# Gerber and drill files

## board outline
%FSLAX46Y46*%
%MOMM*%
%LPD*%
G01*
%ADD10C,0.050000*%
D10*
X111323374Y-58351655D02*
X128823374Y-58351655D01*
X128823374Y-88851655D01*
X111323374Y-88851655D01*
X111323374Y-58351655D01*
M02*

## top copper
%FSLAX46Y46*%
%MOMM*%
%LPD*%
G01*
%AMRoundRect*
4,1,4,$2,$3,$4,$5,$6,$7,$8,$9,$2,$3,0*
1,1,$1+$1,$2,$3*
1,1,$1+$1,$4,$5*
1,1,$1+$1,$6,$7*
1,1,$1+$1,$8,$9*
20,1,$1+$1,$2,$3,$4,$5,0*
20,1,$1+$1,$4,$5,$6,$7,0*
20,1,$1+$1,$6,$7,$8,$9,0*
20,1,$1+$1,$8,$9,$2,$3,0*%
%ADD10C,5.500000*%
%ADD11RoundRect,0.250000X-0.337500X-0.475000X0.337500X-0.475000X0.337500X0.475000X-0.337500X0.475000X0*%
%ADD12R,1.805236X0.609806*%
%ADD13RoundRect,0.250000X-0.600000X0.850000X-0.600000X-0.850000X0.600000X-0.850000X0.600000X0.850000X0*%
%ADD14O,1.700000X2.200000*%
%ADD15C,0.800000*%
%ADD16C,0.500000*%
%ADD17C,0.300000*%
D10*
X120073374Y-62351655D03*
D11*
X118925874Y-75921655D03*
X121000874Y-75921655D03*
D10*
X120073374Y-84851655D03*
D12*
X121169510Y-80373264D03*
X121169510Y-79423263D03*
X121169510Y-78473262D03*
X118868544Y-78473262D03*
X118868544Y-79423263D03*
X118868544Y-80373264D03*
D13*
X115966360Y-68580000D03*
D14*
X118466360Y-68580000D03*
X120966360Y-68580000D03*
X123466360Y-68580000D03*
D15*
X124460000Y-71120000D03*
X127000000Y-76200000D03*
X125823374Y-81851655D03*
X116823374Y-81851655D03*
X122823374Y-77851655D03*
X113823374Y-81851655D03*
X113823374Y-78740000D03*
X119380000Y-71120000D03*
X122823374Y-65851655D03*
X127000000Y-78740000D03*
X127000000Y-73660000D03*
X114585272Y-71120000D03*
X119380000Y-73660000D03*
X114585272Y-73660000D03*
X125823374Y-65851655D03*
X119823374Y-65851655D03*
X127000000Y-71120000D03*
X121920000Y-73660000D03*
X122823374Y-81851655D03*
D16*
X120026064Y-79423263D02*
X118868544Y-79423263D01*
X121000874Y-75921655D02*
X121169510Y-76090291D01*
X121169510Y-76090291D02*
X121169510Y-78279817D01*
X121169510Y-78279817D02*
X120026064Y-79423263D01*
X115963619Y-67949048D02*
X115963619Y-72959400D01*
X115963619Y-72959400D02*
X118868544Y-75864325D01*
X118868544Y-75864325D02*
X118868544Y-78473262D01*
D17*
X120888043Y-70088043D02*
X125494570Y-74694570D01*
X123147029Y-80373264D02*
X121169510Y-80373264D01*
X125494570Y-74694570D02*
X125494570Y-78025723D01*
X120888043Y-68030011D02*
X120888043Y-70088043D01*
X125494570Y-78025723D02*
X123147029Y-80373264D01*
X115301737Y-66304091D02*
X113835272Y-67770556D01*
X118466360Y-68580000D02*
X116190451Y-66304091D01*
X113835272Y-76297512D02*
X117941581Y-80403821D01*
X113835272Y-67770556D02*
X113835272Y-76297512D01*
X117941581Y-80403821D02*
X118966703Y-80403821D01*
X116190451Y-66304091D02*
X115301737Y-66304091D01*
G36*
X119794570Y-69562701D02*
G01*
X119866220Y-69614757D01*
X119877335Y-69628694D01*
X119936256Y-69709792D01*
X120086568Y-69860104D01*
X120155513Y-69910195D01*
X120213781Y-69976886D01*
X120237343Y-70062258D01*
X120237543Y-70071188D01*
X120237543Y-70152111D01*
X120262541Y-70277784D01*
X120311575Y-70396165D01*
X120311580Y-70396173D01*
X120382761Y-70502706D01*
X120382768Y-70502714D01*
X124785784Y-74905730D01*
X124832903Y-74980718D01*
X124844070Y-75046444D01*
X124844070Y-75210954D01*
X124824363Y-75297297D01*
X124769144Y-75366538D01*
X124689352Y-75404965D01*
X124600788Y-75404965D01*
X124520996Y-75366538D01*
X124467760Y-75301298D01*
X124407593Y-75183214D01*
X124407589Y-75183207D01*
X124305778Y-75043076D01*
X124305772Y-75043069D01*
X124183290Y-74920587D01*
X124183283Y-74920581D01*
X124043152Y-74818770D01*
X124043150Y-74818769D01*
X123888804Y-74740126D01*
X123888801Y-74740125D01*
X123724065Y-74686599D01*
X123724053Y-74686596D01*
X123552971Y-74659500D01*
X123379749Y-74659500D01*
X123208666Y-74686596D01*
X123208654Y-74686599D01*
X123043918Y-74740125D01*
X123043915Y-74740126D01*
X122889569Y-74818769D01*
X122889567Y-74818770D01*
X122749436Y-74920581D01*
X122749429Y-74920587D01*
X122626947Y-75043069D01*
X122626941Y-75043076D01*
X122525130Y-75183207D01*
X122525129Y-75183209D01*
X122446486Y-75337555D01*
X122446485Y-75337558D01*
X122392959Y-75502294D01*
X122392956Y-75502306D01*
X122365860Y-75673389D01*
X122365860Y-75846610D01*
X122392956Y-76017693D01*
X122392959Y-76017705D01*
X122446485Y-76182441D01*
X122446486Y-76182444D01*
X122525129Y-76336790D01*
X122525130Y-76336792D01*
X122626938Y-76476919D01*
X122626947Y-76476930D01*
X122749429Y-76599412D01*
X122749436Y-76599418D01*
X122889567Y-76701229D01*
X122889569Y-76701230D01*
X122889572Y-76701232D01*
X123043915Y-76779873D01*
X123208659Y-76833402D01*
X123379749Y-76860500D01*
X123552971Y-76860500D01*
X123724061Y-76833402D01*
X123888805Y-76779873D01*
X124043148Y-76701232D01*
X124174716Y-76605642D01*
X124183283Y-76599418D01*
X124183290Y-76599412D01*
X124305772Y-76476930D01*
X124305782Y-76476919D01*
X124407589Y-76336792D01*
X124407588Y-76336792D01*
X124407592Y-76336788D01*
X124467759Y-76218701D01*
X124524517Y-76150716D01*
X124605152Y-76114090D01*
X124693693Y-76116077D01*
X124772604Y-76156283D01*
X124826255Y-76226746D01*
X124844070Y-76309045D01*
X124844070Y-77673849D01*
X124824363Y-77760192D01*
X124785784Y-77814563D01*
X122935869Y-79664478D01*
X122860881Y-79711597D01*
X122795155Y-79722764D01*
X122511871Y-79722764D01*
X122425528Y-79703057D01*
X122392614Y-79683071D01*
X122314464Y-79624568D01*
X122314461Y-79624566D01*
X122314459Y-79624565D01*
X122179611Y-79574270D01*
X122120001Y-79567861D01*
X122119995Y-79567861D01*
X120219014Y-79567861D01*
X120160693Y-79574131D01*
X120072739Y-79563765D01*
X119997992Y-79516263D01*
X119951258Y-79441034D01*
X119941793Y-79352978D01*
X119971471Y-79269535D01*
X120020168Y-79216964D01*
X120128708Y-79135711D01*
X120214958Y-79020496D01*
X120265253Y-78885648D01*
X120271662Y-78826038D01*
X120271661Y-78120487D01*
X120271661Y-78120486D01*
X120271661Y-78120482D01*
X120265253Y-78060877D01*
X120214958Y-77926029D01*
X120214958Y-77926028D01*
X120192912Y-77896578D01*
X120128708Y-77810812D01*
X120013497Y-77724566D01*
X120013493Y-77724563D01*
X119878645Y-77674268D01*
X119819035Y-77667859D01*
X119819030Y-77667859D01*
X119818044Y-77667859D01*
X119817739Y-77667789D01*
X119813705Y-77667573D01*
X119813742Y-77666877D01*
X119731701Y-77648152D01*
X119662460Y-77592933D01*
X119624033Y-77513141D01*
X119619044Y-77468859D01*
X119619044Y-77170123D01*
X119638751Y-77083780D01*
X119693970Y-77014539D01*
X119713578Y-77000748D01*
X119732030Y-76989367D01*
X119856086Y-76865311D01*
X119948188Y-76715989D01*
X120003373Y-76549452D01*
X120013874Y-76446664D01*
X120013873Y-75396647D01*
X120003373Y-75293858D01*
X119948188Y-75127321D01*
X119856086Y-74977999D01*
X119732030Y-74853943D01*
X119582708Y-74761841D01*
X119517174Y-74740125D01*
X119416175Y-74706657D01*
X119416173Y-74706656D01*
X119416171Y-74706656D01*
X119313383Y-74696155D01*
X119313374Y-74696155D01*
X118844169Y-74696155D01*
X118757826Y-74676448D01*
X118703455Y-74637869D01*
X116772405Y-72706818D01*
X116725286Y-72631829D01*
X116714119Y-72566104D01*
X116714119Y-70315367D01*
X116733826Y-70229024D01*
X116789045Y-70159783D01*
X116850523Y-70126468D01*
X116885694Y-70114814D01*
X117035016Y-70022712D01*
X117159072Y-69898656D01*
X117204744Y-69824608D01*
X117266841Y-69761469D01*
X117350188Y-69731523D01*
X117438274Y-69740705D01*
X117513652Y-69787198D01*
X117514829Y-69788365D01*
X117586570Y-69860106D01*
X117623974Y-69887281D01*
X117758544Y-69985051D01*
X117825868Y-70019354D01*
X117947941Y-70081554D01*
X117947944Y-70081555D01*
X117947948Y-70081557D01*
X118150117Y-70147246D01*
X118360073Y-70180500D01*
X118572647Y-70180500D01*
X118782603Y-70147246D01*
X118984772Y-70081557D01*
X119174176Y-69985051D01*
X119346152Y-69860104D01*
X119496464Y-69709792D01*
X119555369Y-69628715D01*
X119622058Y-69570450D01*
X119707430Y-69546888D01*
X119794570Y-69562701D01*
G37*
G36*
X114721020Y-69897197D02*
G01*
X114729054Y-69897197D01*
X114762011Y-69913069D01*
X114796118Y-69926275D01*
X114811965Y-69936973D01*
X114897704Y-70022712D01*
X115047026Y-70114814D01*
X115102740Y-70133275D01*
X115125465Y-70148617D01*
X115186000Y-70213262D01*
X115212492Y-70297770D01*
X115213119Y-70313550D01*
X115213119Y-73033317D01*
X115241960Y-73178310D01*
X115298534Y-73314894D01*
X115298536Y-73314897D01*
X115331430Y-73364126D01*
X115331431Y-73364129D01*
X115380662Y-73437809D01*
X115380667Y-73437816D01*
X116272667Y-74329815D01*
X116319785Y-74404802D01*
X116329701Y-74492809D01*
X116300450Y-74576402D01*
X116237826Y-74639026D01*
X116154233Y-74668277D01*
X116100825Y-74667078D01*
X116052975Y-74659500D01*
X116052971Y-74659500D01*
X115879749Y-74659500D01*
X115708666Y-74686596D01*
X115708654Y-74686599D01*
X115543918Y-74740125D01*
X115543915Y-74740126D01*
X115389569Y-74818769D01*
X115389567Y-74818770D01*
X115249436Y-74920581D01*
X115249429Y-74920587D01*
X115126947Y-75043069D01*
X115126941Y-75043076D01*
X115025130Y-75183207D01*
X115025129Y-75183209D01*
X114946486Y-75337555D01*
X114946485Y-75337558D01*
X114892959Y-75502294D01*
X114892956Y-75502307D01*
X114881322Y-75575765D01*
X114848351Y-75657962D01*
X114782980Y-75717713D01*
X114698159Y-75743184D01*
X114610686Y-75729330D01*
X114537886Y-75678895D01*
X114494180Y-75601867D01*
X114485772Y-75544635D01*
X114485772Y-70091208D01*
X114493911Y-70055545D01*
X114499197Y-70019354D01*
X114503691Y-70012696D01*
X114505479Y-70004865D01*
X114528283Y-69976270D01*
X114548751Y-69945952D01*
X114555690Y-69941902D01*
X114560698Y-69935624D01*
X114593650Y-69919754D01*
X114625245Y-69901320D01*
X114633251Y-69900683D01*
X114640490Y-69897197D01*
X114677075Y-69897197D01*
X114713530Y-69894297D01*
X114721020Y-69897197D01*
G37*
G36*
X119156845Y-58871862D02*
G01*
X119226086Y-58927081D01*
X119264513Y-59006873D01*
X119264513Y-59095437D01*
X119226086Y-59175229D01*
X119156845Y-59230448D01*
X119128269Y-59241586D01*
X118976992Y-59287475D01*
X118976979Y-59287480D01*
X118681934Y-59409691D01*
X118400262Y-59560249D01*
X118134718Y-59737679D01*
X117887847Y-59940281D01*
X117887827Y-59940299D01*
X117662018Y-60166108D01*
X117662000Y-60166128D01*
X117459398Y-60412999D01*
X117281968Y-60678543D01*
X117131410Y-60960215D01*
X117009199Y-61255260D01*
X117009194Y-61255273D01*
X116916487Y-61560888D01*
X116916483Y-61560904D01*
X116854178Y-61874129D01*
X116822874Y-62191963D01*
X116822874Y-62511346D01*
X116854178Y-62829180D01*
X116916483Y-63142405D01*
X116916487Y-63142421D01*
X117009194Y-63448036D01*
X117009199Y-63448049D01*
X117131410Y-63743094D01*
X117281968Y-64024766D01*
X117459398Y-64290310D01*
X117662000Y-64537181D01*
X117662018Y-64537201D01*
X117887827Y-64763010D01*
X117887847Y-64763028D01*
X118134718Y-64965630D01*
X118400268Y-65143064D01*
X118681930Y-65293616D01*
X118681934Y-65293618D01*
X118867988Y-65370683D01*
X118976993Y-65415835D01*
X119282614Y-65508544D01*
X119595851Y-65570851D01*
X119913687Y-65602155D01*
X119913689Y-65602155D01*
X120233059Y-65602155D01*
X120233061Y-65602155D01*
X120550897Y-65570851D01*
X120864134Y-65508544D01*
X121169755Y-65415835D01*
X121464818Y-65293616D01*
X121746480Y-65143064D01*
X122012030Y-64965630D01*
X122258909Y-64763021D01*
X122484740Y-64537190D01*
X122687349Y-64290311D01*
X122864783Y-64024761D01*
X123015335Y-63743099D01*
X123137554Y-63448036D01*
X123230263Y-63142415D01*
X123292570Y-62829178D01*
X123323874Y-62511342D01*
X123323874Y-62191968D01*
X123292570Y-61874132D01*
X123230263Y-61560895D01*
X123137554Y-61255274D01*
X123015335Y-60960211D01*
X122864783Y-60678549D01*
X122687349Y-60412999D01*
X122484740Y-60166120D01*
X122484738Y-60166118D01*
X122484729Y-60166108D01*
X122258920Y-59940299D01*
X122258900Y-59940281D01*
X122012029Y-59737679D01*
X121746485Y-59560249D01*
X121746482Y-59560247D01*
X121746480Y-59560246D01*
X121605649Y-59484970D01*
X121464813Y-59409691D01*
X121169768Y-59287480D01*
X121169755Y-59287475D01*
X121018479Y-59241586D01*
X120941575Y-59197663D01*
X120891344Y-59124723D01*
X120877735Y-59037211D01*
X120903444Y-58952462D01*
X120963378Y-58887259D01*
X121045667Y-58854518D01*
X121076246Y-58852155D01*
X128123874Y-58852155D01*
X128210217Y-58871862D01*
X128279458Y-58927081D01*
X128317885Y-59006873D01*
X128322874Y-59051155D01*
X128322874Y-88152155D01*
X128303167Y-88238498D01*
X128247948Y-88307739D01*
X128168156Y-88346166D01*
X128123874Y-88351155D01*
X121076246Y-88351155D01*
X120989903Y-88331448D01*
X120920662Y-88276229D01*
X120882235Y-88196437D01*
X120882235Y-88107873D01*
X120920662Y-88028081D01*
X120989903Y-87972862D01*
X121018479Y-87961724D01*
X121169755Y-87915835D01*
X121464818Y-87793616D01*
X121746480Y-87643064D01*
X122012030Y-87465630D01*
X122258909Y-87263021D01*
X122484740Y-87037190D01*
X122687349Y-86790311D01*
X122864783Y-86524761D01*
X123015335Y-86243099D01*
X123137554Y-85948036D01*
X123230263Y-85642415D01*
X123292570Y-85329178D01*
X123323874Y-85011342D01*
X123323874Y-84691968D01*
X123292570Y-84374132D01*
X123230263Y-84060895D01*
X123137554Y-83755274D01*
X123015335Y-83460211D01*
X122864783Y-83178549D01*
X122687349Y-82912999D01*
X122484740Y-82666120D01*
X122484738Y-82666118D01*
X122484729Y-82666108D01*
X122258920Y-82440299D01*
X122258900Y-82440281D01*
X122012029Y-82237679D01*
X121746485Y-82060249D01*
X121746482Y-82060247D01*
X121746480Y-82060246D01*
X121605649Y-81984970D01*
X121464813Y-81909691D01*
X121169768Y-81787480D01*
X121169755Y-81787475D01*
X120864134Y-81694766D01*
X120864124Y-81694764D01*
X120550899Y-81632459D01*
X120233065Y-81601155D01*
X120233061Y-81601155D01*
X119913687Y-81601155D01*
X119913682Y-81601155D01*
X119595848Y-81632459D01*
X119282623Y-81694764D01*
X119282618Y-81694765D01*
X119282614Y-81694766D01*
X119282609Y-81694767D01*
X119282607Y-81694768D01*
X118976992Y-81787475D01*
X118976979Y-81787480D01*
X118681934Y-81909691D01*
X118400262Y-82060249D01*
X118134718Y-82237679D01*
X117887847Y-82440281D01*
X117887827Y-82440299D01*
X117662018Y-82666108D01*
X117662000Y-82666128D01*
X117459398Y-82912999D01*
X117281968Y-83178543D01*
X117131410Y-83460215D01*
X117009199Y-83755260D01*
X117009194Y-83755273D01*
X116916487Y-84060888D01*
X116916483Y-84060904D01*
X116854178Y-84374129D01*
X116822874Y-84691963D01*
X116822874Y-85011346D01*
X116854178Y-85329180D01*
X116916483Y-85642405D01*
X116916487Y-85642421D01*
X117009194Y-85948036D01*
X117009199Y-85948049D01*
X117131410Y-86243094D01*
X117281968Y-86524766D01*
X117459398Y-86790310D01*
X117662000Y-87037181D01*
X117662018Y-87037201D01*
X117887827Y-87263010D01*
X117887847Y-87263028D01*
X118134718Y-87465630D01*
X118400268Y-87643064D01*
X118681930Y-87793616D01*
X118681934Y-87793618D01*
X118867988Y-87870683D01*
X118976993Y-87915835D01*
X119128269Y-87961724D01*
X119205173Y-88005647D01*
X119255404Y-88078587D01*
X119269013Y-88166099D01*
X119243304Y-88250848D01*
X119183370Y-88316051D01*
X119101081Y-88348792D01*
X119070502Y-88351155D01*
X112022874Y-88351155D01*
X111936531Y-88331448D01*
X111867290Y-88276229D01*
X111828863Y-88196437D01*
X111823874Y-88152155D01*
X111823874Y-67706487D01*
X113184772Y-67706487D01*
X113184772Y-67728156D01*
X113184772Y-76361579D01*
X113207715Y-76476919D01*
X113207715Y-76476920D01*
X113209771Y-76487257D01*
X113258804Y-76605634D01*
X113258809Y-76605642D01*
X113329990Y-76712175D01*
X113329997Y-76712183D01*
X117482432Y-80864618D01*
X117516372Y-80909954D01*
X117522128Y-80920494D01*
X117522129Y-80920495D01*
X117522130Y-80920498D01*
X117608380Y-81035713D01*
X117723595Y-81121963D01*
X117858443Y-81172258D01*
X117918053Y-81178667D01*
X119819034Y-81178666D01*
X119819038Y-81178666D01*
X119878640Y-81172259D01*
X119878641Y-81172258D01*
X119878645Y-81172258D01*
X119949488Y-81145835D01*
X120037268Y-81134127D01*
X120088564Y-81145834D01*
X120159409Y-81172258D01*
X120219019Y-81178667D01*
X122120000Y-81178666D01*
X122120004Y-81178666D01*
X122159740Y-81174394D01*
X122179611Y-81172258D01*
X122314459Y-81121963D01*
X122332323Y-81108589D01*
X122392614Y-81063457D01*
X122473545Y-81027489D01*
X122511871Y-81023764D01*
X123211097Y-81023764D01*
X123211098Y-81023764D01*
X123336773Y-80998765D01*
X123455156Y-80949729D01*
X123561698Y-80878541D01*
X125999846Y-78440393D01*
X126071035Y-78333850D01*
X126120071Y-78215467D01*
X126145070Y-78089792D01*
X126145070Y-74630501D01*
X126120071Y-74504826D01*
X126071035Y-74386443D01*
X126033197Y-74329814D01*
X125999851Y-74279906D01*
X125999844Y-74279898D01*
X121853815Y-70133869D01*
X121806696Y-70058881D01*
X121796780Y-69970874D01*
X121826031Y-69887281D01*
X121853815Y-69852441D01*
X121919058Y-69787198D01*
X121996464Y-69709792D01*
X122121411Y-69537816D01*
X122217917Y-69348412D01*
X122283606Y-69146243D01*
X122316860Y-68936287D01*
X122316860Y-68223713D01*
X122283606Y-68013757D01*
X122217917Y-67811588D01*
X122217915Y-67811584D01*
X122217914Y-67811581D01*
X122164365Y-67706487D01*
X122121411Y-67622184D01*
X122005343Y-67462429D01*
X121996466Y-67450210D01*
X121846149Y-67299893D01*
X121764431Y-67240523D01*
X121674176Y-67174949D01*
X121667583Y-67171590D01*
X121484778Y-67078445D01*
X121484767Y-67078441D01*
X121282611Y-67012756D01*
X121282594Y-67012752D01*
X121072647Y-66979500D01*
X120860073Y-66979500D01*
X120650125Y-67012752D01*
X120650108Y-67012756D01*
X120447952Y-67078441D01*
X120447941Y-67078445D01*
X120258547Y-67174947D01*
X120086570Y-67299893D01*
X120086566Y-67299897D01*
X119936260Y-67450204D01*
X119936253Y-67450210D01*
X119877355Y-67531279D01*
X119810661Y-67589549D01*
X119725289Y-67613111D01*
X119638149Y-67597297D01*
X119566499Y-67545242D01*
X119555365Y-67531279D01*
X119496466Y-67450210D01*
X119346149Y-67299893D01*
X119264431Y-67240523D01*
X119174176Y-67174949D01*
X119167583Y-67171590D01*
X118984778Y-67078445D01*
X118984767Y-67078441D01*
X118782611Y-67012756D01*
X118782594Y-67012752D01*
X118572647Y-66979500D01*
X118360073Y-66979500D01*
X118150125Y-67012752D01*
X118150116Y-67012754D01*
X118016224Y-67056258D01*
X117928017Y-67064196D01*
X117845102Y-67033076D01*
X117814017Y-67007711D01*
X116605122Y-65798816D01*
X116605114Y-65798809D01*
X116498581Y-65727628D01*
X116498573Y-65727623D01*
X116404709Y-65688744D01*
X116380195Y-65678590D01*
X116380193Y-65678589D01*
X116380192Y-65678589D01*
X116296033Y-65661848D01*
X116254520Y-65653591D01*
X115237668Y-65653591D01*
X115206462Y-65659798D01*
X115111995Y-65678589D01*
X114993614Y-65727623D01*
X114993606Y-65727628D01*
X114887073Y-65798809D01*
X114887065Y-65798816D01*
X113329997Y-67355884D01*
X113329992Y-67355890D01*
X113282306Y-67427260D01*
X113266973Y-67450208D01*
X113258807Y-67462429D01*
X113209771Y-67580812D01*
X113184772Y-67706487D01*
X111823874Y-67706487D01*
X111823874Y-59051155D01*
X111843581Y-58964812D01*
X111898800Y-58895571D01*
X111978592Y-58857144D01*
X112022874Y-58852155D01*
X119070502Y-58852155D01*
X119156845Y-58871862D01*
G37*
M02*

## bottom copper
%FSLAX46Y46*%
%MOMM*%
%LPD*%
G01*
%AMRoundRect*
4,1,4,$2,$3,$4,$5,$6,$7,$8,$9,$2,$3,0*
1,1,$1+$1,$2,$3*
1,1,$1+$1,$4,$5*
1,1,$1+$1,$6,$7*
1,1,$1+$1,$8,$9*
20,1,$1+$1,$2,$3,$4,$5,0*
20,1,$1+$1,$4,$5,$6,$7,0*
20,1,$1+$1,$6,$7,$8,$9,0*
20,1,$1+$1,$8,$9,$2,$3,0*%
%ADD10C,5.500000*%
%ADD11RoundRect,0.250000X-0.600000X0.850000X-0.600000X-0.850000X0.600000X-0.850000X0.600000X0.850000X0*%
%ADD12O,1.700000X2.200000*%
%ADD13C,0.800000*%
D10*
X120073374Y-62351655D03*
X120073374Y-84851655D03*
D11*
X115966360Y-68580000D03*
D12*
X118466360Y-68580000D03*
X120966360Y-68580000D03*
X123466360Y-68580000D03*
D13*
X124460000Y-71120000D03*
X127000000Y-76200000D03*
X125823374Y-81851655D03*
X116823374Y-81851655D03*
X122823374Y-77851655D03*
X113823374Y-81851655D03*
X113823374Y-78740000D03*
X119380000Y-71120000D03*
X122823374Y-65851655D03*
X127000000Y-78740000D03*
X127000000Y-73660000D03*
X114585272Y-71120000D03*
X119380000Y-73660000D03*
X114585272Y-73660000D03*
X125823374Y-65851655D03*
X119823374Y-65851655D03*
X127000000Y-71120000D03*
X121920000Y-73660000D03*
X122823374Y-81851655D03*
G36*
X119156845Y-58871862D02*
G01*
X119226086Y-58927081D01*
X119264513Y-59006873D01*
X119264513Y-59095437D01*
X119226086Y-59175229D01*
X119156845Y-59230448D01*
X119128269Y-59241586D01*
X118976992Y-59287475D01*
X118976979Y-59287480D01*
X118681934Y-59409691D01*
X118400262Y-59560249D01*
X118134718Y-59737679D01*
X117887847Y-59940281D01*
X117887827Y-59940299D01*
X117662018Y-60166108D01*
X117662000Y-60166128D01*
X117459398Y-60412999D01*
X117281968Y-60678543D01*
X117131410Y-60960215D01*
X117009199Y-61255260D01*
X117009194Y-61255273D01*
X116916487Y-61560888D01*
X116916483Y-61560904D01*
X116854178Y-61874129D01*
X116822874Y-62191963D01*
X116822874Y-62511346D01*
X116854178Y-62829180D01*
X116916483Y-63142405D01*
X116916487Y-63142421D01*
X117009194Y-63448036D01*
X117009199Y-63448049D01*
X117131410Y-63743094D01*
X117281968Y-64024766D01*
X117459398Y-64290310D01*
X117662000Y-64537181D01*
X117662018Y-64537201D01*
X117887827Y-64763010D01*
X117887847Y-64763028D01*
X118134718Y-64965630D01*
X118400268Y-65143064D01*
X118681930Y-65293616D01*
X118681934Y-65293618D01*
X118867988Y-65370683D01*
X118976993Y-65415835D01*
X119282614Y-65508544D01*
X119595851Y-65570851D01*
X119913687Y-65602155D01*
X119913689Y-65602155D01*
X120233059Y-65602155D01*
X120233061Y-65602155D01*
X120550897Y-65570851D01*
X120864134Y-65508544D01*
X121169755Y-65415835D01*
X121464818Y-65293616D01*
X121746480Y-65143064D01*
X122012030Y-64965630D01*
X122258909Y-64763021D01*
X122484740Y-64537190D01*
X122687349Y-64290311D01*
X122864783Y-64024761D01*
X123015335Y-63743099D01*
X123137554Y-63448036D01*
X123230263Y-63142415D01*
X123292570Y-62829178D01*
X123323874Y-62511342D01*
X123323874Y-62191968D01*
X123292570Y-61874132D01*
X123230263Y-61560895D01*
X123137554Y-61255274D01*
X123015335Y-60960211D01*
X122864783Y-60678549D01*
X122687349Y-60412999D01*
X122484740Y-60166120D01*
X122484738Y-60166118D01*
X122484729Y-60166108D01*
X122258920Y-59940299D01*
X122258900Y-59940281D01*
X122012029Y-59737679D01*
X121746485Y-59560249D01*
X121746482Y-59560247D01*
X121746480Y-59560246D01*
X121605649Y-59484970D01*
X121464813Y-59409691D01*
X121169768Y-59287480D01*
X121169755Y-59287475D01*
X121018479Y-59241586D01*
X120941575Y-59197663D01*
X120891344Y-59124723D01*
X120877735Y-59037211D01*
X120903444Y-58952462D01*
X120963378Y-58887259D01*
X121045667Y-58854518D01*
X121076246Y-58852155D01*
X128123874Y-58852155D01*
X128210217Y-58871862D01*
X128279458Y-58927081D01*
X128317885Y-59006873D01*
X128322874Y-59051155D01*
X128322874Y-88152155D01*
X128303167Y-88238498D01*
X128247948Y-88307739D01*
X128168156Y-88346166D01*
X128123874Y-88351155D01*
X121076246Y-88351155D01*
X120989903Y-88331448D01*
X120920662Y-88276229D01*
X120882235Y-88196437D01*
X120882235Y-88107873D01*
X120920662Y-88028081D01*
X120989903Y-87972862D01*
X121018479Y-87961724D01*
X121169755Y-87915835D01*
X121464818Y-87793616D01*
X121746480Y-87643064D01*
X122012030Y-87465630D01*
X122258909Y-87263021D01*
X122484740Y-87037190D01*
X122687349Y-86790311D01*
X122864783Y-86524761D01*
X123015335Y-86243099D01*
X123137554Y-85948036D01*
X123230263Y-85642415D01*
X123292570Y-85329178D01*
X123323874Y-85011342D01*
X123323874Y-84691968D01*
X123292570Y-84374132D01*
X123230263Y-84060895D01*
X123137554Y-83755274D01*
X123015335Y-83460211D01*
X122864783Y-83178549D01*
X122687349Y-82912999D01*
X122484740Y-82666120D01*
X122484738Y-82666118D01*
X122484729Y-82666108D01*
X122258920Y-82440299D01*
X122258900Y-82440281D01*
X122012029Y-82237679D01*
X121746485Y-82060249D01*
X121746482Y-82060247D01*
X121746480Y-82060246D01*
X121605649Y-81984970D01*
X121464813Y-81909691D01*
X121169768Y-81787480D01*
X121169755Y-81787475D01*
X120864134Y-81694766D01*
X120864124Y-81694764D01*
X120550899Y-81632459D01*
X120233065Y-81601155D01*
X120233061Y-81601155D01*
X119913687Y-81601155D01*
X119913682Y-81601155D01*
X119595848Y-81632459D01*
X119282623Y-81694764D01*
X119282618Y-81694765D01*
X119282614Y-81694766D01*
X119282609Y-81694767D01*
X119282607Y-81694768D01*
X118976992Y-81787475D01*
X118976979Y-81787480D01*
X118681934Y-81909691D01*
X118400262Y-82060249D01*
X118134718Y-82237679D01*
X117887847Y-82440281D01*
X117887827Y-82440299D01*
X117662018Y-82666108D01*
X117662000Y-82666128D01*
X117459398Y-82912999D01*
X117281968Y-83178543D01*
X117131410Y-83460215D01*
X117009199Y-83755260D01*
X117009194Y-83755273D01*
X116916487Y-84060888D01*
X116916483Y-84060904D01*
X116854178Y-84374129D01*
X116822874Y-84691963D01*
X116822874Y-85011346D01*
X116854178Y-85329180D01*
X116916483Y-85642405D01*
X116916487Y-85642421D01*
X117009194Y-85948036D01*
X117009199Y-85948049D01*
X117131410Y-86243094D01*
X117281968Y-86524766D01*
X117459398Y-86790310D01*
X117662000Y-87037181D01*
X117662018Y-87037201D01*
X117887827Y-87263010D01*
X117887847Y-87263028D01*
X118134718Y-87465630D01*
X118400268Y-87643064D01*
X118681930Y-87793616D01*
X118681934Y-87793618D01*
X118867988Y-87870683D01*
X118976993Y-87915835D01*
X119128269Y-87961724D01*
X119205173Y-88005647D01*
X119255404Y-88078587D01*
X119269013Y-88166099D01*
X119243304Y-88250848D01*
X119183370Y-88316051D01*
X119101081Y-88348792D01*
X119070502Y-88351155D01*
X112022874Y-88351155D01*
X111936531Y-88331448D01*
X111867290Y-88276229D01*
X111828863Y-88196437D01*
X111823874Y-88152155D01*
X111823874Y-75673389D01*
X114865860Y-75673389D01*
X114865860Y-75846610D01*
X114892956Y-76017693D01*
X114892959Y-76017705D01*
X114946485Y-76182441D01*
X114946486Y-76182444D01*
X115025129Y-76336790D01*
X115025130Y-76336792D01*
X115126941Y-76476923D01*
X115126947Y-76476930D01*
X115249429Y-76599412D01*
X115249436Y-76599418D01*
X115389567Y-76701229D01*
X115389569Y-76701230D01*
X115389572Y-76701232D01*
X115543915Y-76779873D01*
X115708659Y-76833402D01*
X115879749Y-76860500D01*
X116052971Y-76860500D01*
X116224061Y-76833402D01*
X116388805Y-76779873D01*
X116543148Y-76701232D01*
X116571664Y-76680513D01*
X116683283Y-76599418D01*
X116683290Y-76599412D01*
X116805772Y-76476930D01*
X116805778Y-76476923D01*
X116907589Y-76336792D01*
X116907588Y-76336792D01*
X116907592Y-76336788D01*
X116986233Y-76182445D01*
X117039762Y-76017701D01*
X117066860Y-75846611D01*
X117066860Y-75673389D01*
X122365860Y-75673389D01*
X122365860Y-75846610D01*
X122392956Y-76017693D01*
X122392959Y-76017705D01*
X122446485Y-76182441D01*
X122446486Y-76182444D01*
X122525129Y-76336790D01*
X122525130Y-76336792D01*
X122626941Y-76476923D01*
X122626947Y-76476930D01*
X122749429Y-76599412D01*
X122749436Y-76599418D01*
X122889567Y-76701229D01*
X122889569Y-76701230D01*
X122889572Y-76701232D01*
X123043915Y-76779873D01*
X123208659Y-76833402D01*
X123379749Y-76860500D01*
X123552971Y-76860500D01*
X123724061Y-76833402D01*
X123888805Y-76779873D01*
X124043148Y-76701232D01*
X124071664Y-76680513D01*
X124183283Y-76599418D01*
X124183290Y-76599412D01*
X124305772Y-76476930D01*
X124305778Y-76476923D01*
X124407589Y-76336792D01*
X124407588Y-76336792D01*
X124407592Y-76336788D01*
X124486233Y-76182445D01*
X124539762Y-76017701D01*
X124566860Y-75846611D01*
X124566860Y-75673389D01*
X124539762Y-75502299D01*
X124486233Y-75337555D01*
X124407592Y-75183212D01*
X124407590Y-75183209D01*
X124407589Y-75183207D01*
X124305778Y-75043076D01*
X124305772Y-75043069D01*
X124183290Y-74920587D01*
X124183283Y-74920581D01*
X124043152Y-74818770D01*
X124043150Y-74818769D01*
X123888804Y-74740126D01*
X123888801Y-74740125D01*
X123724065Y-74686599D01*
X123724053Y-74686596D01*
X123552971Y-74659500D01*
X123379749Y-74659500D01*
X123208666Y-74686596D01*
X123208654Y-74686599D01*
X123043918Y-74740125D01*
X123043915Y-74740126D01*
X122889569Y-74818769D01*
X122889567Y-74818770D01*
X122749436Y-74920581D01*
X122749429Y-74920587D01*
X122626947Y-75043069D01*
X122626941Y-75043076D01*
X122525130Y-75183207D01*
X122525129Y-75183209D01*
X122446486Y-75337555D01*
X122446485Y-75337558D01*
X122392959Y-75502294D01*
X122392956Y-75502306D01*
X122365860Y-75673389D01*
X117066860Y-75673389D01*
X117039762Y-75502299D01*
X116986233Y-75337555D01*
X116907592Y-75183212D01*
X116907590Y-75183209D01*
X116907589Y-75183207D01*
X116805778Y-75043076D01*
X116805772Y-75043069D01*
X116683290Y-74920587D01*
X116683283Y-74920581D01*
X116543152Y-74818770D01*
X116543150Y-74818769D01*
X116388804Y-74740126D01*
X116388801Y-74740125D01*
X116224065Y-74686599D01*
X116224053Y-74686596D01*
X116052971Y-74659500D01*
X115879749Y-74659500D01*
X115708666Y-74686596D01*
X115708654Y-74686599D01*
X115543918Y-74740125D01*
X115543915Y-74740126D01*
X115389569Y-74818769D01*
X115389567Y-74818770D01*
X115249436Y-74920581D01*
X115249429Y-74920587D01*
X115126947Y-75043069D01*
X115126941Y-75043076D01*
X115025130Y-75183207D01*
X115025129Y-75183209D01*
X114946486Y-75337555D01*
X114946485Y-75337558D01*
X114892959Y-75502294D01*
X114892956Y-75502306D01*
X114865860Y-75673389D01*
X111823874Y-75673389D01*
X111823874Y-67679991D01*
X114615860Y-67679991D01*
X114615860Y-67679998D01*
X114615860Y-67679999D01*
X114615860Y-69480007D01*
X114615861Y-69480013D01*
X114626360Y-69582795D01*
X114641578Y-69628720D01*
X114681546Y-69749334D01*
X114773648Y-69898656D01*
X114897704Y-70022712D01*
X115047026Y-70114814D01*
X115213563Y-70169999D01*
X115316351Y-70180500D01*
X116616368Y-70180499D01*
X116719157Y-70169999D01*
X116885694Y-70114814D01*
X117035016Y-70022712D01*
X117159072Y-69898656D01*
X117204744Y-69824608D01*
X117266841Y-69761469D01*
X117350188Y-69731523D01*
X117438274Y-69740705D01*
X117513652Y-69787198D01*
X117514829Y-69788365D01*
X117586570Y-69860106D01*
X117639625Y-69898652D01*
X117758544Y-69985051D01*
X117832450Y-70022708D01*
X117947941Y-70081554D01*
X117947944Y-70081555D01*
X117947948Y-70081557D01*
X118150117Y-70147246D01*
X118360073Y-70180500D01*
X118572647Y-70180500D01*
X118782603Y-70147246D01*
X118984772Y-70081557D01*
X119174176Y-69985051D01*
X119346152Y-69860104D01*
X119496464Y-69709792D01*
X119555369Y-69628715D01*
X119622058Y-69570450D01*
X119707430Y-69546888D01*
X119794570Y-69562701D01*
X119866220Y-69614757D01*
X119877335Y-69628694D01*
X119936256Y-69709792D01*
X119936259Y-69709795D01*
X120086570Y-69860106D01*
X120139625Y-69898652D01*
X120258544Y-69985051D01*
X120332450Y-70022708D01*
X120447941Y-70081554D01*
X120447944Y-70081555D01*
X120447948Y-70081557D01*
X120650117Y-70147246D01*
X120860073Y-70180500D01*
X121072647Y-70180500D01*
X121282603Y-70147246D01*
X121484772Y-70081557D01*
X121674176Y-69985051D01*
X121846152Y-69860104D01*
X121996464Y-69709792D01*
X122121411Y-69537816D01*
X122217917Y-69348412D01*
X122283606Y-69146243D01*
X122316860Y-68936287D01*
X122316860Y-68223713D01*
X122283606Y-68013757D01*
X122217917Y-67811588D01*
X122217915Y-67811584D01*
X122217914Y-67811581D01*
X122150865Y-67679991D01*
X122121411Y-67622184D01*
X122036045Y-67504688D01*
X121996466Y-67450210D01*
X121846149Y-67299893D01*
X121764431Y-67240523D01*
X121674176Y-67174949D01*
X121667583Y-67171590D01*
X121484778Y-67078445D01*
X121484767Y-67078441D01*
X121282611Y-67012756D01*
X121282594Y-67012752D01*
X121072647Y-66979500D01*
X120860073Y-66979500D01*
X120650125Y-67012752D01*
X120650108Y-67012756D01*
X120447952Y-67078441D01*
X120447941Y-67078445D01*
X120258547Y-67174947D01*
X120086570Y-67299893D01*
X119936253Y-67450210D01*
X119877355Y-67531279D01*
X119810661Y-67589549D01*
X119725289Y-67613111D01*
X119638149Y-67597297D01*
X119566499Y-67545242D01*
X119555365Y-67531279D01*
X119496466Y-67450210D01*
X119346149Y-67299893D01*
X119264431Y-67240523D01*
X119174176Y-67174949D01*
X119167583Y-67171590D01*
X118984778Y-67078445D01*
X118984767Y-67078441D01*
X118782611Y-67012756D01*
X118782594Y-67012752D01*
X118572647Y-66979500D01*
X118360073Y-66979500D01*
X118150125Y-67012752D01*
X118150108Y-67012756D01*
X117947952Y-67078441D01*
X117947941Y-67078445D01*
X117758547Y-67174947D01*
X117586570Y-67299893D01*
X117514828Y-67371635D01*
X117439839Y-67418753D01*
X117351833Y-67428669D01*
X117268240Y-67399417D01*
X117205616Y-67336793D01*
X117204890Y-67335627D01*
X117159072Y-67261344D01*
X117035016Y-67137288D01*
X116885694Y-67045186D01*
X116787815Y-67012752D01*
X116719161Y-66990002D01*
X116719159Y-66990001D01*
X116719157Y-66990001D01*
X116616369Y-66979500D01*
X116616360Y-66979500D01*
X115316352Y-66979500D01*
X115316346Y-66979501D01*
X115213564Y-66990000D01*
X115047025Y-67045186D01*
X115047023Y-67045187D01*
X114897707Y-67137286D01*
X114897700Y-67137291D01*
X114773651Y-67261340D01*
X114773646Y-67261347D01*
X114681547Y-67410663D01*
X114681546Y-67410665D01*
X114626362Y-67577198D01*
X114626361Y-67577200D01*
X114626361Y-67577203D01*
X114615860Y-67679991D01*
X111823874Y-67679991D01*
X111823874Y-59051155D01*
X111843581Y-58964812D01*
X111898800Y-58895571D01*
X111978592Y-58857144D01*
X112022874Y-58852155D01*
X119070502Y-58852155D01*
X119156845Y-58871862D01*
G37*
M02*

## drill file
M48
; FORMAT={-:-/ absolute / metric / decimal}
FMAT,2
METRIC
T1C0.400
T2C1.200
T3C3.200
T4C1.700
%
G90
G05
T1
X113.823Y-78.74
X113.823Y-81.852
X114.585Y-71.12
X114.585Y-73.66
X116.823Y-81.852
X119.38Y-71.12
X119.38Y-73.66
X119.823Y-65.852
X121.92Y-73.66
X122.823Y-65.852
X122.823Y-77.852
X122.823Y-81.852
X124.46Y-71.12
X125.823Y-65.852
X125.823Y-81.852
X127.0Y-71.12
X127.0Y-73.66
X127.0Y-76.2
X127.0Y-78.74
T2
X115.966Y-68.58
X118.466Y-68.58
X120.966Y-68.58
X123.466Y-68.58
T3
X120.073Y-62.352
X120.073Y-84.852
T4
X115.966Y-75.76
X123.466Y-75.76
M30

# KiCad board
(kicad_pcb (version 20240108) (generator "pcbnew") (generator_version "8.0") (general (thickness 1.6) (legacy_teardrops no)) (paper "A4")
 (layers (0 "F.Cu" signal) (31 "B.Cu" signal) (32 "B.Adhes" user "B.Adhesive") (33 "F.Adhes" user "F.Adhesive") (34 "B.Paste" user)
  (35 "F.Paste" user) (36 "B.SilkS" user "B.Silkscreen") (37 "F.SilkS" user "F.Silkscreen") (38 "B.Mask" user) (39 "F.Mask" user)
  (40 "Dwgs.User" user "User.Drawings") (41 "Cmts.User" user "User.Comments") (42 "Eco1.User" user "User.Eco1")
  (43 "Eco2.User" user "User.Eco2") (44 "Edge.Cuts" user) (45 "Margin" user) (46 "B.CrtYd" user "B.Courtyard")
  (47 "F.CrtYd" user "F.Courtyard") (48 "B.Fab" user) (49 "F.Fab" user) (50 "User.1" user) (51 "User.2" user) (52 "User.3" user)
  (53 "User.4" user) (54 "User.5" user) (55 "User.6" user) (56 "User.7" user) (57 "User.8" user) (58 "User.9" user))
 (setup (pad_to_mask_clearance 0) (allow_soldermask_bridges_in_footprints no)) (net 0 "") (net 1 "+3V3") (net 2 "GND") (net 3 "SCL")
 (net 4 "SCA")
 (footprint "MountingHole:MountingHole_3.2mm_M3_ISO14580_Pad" (layer "F.Cu") (at 120.073374 62.351655)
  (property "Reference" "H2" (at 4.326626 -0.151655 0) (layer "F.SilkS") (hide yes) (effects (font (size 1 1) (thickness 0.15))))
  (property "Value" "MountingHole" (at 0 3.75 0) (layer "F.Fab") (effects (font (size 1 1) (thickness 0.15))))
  (pad "1" thru_hole circle (at 0 0) (size 5.5 5.5) (drill 3.2) (layers "*.Cu" "*.Mask") (remove_unused_layers no)))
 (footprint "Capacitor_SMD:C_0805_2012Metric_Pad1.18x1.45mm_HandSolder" (layer "F.Cu") (at 119.963374 75.921655)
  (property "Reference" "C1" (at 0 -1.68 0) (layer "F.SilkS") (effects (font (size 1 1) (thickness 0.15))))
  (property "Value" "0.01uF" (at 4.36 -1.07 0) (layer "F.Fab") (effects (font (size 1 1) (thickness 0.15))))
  (pad "1" smd roundrect (at -1.0375 0) (size 1.175 1.45) (layers "F.Cu" "F.Paste" "F.Mask") (roundrect_rratio 0.212766) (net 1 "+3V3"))
  (pad "2" smd roundrect (at 1.0375 0) (size 1.175 1.45) (layers "F.Cu" "F.Paste" "F.Mask") (roundrect_rratio 0.212766) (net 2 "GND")))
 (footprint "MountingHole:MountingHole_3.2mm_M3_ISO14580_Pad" (layer "F.Cu") (at 120.073374 84.851655)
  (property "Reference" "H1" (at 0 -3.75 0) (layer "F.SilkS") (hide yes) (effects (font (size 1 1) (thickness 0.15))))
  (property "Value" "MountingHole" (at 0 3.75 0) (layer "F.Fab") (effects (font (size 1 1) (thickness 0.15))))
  (pad "1" thru_hole circle (at 0 0) (size 5.5 5.5) (drill 3.2) (layers "*.Cu" "*.Mask") (remove_unused_layers no)))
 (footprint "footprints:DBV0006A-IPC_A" (layer "F.Cu") (at 120.019027 79.423263 180)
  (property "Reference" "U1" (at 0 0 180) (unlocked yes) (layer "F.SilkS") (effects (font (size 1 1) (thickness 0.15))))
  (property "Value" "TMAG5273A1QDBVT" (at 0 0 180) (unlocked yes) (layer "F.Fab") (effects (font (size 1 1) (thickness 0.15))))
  (pad "1" smd rect (at -1.150483 -0.950001 180) (size 1.805236 0.609806) (layers "F.Cu" "F.Paste" "F.Mask") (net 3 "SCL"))
  (pad "2" smd rect (at -1.150483 0 180) (size 1.805236 0.609806) (layers "F.Cu" "F.Paste" "F.Mask") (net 2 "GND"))
  (pad "3" smd rect (at -1.150483 0.950001 180) (size 1.805236 0.609806) (layers "F.Cu" "F.Paste" "F.Mask") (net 2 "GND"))
  (pad "4" smd rect (at 1.150483 0.950001 180) (size 1.805236 0.609806) (layers "F.Cu" "F.Paste" "F.Mask") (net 1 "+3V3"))
  (pad "5" smd rect (at 1.150483 0 180) (size 1.805236 0.609806) (layers "F.Cu" "F.Paste" "F.Mask") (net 2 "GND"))
  (pad "6" smd rect (at 1.150483 -0.950001 180) (size 1.805236 0.609806) (layers "F.Cu" "F.Paste" "F.Mask") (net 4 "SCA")))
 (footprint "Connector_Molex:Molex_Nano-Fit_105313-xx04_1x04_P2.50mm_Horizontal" (layer "B.Cu") (at 115.96636 68.58 -90)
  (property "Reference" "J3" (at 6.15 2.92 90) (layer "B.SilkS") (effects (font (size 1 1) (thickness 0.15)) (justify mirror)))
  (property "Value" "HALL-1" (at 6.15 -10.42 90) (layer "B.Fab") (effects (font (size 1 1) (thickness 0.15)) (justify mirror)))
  (pad "" np_thru_hole circle (at 7.18 -7.5 270) (size 1.7 1.7) (drill 1.7) (layers "*.Cu" "*.Mask"))
  (pad "" np_thru_hole circle (at 7.18 0 270) (size 1.7 1.7) (drill 1.7) (layers "*.Cu" "*.Mask"))
  (pad "1" thru_hole roundrect (at 0 0 270) (size 2.2 1.7) (drill 1.2) (layers "*.Cu" "*.Mask") (remove_unused_layers no)
   (roundrect_rratio 0.147059) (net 1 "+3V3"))
  (pad "2" thru_hole oval (at 0 -2.5 270) (size 2.2 1.7) (drill 1.2) (layers "*.Cu" "*.Mask") (remove_unused_layers no) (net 4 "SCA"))
  (pad "3" thru_hole oval (at 0 -5 270) (size 2.2 1.7) (drill 1.2) (layers "*.Cu" "*.Mask") (remove_unused_layers no) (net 3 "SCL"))
  (pad "4" thru_hole oval (at 0 -7.5 270) (size 2.2 1.7) (drill 1.2) (layers "*.Cu" "*.Mask") (remove_unused_layers no) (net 2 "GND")))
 (gr_rect (start 111.323374 58.351655) (end 128.823374 88.851655) (stroke (width 0.05) (type default)) (fill none) (layer "Edge.Cuts"))
 (segment (start 120.026064 79.423263) (end 118.868544 79.423263) (width 0.5) (layer "F.Cu") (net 2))
 (segment (start 121.000874 75.921655) (end 121.16951 76.090291) (width 0.5) (layer "F.Cu") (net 2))
 (segment (start 121.16951 76.090291) (end 121.16951 78.279817) (width 0.5) (layer "F.Cu") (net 2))
 (segment (start 121.16951 78.279817) (end 120.026064 79.423263) (width 0.5) (layer "F.Cu") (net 2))
 (via (at 124.46 71.12) (size 0.8) (drill 0.4) (layers "F.Cu" "B.Cu") (free yes) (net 2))
 (via (at 127 76.2) (size 0.8) (drill 0.4) (layers "F.Cu" "B.Cu") (free yes) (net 2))
 (via (at 125.823374 81.851655) (size 0.8) (drill 0.4) (layers "F.Cu" "B.Cu") (free yes) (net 2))
 (via (at 116.823374 81.851655) (size 0.8) (drill 0.4) (layers "F.Cu" "B.Cu") (free yes) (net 2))
 (via (at 122.823374 77.851655) (size 0.8) (drill 0.4) (layers "F.Cu" "B.Cu") (free yes) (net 2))
 (via (at 113.823374 81.851655) (size 0.8) (drill 0.4) (layers "F.Cu" "B.Cu") (free yes) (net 2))
 (via (at 113.823374 78.74) (size 0.8) (drill 0.4) (layers "F.Cu" "B.Cu") (free yes) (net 2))
 (via (at 119.38 71.12) (size 0.8) (drill 0.4) (layers "F.Cu" "B.Cu") (free yes) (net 2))
 (via (at 122.823374 65.851655) (size 0.8) (drill 0.4) (layers "F.Cu" "B.Cu") (free yes) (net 2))
 (via (at 127 78.74) (size 0.8) (drill 0.4) (layers "F.Cu" "B.Cu") (free yes) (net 2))
 (via (at 127 73.66) (size 0.8) (drill 0.4) (layers "F.Cu" "B.Cu") (free yes) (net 2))
 (via (at 114.585272 71.12) (size 0.8) (drill 0.4) (layers "F.Cu" "B.Cu") (free yes) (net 2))
 (via (at 119.38 73.66) (size 0.8) (drill 0.4) (layers "F.Cu" "B.Cu") (free yes) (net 2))
 (via (at 114.585272 73.66) (size 0.8) (drill 0.4) (layers "F.Cu" "B.Cu") (free yes) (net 2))
 (via (at 125.823374 65.851655) (size 0.8) (drill 0.4) (layers "F.Cu" "B.Cu") (free yes) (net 2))
 (via (at 119.823374 65.851655) (size 0.8) (drill 0.4) (layers "F.Cu" "B.Cu") (free yes) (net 2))
 (via (at 127 71.12) (size 0.8) (drill 0.4) (layers "F.Cu" "B.Cu") (free yes) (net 2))
 (via (at 121.92 73.66) (size 0.8) (drill 0.4) (layers "F.Cu" "B.Cu") (free yes) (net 2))
 (via (at 122.823374 81.851655) (size 0.8) (drill 0.4) (layers "F.Cu" "B.Cu") (free yes) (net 2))
 (segment (start 115.963619 67.949048) (end 115.963619 72.9594) (width 0.5) (layer "F.Cu") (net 1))
 (segment (start 115.963619 72.9594) (end 118.868544 75.864325) (width 0.5) (layer "F.Cu") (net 1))
 (segment (start 118.868544 75.864325) (end 118.868544 78.473262) (width 0.5) (layer "F.Cu") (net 1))
 (segment (start 120.888043 70.088043) (end 125.49457 74.69457) (width 0.3) (layer "F.Cu") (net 3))
 (segment (start 123.147029 80.373264) (end 121.16951 80.373264) (width 0.3) (layer "F.Cu") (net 3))
 (segment (start 125.49457 74.69457) (end 125.49457 78.025723) (width 0.3) (layer "F.Cu") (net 3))
 (segment (start 120.888043 68.030011) (end 120.888043 70.088043) (width 0.3) (layer "F.Cu") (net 3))
 (segment (start 125.49457 78.025723) (end 123.147029 80.373264) (width 0.3) (layer "F.Cu") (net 3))
 (segment (start 115.301737 66.304091) (end 113.835272 67.770556) (width 0.3) (layer "F.Cu") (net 4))
 (segment (start 118.46636 68.58) (end 116.190451 66.304091) (width 0.3) (layer "F.Cu") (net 4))
 (segment (start 113.835272 76.297512) (end 117.941581 80.403821) (width 0.3) (layer "F.Cu") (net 4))
 (segment (start 113.835272 67.770556) (end 113.835272 76.297512) (width 0.3) (layer "F.Cu") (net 4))
 (segment (start 117.941581 80.403821) (end 118.966703 80.403821) (width 0.3) (layer "F.Cu") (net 4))
 (segment (start 116.190451 66.304091) (end 115.301737 66.304091) (width 0.3) (layer "F.Cu") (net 4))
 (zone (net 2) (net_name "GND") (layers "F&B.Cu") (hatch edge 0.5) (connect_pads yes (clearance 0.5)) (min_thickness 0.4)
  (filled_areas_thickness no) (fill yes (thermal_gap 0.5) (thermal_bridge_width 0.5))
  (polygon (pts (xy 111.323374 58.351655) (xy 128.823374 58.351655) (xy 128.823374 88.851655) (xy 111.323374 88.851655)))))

